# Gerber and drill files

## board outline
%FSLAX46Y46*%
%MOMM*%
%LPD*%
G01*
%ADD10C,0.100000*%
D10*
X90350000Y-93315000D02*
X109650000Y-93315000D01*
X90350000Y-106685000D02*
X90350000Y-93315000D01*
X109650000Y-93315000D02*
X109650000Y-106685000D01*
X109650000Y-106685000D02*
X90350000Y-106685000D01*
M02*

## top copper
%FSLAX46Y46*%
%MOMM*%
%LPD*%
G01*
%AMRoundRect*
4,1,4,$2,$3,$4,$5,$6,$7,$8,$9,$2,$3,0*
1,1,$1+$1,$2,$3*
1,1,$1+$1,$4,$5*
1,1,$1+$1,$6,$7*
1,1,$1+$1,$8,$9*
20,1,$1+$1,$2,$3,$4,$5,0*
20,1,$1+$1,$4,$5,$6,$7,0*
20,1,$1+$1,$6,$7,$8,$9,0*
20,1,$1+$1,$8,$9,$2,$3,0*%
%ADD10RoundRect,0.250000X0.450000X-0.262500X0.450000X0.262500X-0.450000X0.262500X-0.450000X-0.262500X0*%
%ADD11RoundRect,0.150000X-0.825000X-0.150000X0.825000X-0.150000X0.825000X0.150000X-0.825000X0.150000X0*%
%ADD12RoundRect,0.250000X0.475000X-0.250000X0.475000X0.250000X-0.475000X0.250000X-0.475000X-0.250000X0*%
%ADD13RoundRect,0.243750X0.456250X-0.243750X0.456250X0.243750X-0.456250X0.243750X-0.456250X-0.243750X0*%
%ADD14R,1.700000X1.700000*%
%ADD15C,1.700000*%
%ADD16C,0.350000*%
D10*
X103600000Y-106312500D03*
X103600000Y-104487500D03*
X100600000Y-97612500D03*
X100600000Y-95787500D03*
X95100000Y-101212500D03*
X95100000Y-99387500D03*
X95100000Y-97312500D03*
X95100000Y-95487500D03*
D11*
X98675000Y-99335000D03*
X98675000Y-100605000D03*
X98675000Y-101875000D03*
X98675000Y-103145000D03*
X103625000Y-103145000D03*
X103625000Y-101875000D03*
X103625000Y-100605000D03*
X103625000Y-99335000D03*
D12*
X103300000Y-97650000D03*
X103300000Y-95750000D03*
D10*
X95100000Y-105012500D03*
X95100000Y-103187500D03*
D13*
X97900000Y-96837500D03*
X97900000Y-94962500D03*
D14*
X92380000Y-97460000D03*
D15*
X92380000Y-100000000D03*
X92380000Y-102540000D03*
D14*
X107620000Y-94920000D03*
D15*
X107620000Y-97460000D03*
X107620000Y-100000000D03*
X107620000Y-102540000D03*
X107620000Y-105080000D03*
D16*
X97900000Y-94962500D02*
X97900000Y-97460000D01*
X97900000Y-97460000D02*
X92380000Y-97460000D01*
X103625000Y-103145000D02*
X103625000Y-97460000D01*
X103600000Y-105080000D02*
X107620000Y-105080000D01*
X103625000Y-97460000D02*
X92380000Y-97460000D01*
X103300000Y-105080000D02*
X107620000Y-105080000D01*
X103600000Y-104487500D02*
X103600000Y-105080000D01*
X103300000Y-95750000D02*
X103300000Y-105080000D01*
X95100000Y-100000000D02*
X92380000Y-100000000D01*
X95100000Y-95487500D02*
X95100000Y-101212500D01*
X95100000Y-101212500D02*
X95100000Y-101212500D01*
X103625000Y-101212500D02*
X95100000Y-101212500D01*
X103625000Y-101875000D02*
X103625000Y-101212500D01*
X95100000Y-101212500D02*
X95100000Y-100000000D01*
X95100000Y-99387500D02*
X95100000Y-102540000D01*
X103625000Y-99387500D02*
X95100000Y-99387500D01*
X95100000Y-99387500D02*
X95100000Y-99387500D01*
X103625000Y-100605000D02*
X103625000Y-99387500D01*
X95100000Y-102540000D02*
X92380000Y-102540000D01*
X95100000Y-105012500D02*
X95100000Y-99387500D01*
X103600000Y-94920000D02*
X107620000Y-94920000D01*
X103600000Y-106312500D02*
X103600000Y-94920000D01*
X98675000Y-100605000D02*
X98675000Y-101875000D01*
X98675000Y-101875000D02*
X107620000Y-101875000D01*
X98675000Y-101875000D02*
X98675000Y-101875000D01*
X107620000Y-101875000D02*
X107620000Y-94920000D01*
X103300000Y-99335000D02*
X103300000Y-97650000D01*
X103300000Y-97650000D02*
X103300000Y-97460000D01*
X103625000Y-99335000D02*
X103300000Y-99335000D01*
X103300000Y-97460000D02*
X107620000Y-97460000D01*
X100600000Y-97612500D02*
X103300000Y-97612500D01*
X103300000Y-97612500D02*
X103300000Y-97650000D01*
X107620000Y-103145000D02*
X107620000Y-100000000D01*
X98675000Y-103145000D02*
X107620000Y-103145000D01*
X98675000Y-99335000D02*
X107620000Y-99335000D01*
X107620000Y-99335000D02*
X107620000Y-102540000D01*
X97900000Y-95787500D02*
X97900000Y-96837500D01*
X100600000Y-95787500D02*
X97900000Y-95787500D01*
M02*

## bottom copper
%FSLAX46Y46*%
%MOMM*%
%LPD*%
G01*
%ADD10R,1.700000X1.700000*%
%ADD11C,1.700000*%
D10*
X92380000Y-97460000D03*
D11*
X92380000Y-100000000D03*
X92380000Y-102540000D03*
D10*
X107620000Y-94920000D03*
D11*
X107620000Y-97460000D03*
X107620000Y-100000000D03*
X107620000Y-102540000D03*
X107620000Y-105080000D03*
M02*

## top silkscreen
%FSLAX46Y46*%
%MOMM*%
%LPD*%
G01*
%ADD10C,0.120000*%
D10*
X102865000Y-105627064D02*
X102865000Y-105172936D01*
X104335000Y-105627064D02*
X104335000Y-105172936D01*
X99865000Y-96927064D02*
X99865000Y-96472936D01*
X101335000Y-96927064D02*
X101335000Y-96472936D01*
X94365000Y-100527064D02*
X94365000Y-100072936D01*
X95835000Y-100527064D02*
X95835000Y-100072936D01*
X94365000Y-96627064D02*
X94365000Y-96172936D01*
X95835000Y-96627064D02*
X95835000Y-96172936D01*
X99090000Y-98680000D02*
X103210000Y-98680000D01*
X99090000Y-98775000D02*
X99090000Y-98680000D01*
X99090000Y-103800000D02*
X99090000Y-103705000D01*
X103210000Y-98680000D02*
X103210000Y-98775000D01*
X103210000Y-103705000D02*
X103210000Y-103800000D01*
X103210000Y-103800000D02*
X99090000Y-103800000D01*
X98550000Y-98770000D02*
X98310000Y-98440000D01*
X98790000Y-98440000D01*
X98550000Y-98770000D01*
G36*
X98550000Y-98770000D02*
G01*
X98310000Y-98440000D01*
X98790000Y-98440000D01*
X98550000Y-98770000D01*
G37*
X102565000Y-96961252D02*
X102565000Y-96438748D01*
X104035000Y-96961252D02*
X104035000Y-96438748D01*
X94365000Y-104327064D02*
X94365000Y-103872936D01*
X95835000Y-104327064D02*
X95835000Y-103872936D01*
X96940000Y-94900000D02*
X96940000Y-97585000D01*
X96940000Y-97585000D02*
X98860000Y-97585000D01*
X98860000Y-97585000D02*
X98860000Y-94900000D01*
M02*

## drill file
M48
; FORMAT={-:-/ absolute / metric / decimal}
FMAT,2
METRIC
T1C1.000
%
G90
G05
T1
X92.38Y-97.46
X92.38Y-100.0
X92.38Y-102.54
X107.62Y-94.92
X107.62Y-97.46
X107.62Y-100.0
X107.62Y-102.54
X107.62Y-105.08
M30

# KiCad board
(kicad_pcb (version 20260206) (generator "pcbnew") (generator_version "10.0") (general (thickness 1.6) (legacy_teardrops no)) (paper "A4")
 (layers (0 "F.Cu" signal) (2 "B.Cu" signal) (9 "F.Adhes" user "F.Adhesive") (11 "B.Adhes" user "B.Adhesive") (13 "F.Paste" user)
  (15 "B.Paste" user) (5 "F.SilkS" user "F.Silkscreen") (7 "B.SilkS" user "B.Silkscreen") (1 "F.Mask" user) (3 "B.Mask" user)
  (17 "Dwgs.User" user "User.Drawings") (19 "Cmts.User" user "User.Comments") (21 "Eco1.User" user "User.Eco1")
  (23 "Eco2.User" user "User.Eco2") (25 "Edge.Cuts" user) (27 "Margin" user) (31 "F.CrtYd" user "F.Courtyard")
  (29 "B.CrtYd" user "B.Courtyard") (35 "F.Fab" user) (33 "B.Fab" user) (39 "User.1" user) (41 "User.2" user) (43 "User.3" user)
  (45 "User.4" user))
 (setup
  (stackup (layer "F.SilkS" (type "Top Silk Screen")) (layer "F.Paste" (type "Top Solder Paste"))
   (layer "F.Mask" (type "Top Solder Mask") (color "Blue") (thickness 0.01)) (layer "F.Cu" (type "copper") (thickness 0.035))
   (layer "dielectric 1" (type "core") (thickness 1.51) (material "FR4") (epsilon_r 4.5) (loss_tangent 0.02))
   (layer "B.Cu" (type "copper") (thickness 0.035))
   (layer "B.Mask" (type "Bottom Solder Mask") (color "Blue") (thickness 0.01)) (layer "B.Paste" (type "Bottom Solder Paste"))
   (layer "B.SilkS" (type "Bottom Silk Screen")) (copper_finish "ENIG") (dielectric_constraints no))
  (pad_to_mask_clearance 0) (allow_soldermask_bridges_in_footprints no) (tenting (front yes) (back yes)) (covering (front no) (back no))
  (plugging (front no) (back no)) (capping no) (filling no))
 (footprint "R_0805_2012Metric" (layer "F.Cu") (at 103.6 105.4 90)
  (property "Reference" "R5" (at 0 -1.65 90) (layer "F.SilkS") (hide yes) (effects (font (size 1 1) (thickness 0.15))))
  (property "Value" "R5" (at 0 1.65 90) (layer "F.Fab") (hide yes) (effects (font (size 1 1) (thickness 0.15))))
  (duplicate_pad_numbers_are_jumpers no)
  (fp_line (start -0.227064 -0.735) (end 0.227064 -0.735) (stroke (width 0.12) (type solid)) (layer "F.SilkS"))
  (fp_line (start -0.227064 0.735) (end 0.227064 0.735) (stroke (width 0.12) (type solid)) (layer "F.SilkS"))
  (pad "1" smd roundrect (at -0.9125 0 90) (size 1.025 1.4) (layers "F.Cu" "F.Mask" "F.Paste") (roundrect_rratio 0.243902) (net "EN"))
  (pad "2" smd roundrect (at 0.9125 0 90) (size 1.025 1.4) (layers "F.Cu" "F.Mask" "F.Paste") (roundrect_rratio 0.243902) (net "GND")))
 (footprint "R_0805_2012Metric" (layer "F.Cu") (at 100.6 96.7 90)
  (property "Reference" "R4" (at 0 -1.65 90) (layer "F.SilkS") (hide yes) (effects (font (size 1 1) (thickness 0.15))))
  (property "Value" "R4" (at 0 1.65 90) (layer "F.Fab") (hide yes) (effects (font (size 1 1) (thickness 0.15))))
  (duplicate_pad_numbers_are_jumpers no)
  (fp_line (start -0.227064 -0.735) (end 0.227064 -0.735) (stroke (width 0.12) (type solid)) (layer "F.SilkS"))
  (fp_line (start -0.227064 0.735) (end 0.227064 0.735) (stroke (width 0.12) (type solid)) (layer "F.SilkS"))
  (pad "1" smd roundrect (at -0.9125 0 90) (size 1.025 1.4) (layers "F.Cu" "F.Mask" "F.Paste") (roundrect_rratio 0.243902) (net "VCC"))
  (pad "2" smd roundrect (at 0.9125 0 90) (size 1.025 1.4) (layers "F.Cu" "F.Mask" "F.Paste") (roundrect_rratio 0.243902) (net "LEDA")))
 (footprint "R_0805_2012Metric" (layer "F.Cu") (at 95.1 100.3 90)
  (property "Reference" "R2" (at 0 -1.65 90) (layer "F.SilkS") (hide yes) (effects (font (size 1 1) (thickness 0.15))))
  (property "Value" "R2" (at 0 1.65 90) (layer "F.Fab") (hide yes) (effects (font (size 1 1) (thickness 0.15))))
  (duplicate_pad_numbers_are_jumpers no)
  (fp_line (start -0.227064 -0.735) (end 0.227064 -0.735) (stroke (width 0.12) (type solid)) (layer "F.SilkS"))
  (fp_line (start -0.227064 0.735) (end 0.227064 0.735) (stroke (width 0.12) (type solid)) (layer "F.SilkS"))
  (pad "1" smd roundrect (at -0.9125 0 90) (size 1.025 1.4) (layers "F.Cu" "F.Mask" "F.Paste") (roundrect_rratio 0.243902) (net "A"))
  (pad "2" smd roundrect (at 0.9125 0 90) (size 1.025 1.4) (layers "F.Cu" "F.Mask" "F.Paste") (roundrect_rratio 0.243902) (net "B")))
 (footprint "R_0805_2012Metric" (layer "F.Cu") (at 95.1 96.4 90)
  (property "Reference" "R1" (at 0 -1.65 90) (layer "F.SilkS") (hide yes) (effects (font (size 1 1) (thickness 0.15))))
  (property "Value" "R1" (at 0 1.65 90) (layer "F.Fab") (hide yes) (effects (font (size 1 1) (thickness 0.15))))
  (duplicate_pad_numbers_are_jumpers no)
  (fp_line (start -0.227064 -0.735) (end 0.227064 -0.735) (stroke (width 0.12) (type solid)) (layer "F.SilkS"))
  (fp_line (start -0.227064 0.735) (end 0.227064 0.735) (stroke (width 0.12) (type solid)) (layer "F.SilkS"))
  (pad "1" smd roundrect (at -0.9125 0 90) (size 1.025 1.4) (layers "F.Cu" "F.Mask" "F.Paste") (roundrect_rratio 0.243902) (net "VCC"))
  (pad "2" smd roundrect (at 0.9125 0 90) (size 1.025 1.4) (layers "F.Cu" "F.Mask" "F.Paste") (roundrect_rratio 0.243902) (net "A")))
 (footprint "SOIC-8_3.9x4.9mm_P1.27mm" (layer "F.Cu") (at 101.15 101.24)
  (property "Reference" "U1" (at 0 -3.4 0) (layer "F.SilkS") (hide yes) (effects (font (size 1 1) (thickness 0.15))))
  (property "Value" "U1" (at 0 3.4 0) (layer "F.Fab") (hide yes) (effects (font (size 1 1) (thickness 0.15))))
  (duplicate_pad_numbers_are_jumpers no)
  (fp_line (start -2.06 -2.56) (end 2.06 -2.56) (stroke (width 0.12) (type solid)) (layer "F.SilkS"))
  (fp_line (start -2.06 -2.465) (end -2.06 -2.56) (stroke (width 0.12) (type solid)) (layer "F.SilkS"))
  (fp_line (start -2.06 2.56) (end -2.06 2.465) (stroke (width 0.12) (type solid)) (layer "F.SilkS"))
  (fp_line (start 2.06 -2.56) (end 2.06 -2.465) (stroke (width 0.12) (type solid)) (layer "F.SilkS"))
  (fp_line (start 2.06 2.465) (end 2.06 2.56) (stroke (width 0.12) (type solid)) (layer "F.SilkS"))
  (fp_line (start 2.06 2.56) (end -2.06 2.56) (stroke (width 0.12) (type solid)) (layer "F.SilkS"))
  (fp_poly (pts (xy -2.6 -2.47) (xy -2.84 -2.8) (xy -2.36 -2.8)) (stroke (width 0.12) (type solid)) (fill yes) (layer "F.SilkS"))
  (pad "1" smd roundrect (at -2.475 -1.905) (size 1.95 0.6) (layers "F.Cu" "F.Mask" "F.Paste") (roundrect_rratio 0.25) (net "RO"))
  (pad "2" smd roundrect (at -2.475 -0.635) (size 1.95 0.6) (layers "F.Cu" "F.Mask" "F.Paste") (roundrect_rratio 0.25) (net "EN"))
  (pad "3" smd roundrect (at -2.475 0.635) (size 1.95 0.6) (layers "F.Cu" "F.Mask" "F.Paste") (roundrect_rratio 0.25) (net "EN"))
  (pad "4" smd roundrect (at -2.475 1.905) (size 1.95 0.6) (layers "F.Cu" "F.Mask" "F.Paste") (roundrect_rratio 0.25) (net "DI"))
  (pad "5" smd roundrect (at 2.475 1.905) (size 1.95 0.6) (layers "F.Cu" "F.Mask" "F.Paste") (roundrect_rratio 0.25) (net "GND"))
  (pad "6" smd roundrect (at 2.475 0.635) (size 1.95 0.6) (layers "F.Cu" "F.Mask" "F.Paste") (roundrect_rratio 0.25) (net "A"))
  (pad "7" smd roundrect (at 2.475 -0.635) (size 1.95 0.6) (layers "F.Cu" "F.Mask" "F.Paste") (roundrect_rratio 0.25) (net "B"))
  (pad "8" smd roundrect (at 2.475 -1.905) (size 1.95 0.6) (layers "F.Cu" "F.Mask" "F.Paste") (roundrect_rratio 0.25) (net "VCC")))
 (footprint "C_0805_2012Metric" (layer "F.Cu") (at 103.3 96.7 90)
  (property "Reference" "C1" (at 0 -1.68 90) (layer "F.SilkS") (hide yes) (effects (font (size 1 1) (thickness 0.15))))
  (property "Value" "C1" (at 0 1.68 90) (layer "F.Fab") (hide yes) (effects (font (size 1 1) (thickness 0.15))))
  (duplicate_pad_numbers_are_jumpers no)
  (fp_line (start -0.261252 -0.735) (end 0.261252 -0.735) (stroke (width 0.12) (type solid)) (layer "F.SilkS"))
  (fp_line (start -0.261252 0.735) (end 0.261252 0.735) (stroke (width 0.12) (type solid)) (layer "F.SilkS"))
  (pad "1" smd roundrect (at -0.95 0 90) (size 1 1.45) (layers "F.Cu" "F.Mask" "F.Paste") (roundrect_rratio 0.25) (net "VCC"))
  (pad "2" smd roundrect (at 0.95 0 90) (size 1 1.45) (layers "F.Cu" "F.Mask" "F.Paste") (roundrect_rratio 0.25) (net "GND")))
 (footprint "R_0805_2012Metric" (layer "F.Cu") (at 95.1 104.1 90)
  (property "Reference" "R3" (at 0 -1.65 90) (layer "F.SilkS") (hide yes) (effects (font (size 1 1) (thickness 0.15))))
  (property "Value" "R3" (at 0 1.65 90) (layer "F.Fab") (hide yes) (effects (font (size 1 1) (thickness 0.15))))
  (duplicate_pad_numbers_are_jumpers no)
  (fp_line (start -0.227064 -0.735) (end 0.227064 -0.735) (stroke (width 0.12) (type solid)) (layer "F.SilkS"))
  (fp_line (start -0.227064 0.735) (end 0.227064 0.735) (stroke (width 0.12) (type solid)) (layer "F.SilkS"))
  (pad "1" smd roundrect (at -0.9125 0 90) (size 1.025 1.4) (layers "F.Cu" "F.Mask" "F.Paste") (roundrect_rratio 0.243902) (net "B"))
  (pad "2" smd roundrect (at 0.9125 0 90) (size 1.025 1.4) (layers "F.Cu" "F.Mask" "F.Paste") (roundrect_rratio 0.243902) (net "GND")))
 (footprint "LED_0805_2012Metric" (layer "F.Cu") (at 97.9 95.9 90)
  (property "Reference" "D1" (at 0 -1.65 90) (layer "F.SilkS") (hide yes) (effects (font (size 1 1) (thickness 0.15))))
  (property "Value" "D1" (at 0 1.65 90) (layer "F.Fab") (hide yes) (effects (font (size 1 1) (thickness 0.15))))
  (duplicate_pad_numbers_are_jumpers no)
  (fp_line (start 1 -0.96) (end -1.685 -0.96) (stroke (width 0.12) (type solid)) (layer "F.SilkS"))
  (fp_line (start -1.685 -0.96) (end -1.685 0.96) (stroke (width 0.12) (type solid)) (layer "F.SilkS"))
  (fp_line (start -1.685 0.96) (end 1 0.96) (stroke (width 0.12) (type solid)) (layer "F.SilkS"))
  (pad "1" smd roundrect (at -0.9375 0 90) (size 0.975 1.4) (layers "F.Cu" "F.Mask" "F.Paste") (roundrect_rratio 0.25) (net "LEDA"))
  (pad "2" smd roundrect (at 0.9375 0 90) (size 0.975 1.4) (layers "F.Cu" "F.Mask" "F.Paste") (roundrect_rratio 0.25) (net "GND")))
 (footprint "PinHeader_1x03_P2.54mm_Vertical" (layer "B.Cu") (at 92.38 97.46 180)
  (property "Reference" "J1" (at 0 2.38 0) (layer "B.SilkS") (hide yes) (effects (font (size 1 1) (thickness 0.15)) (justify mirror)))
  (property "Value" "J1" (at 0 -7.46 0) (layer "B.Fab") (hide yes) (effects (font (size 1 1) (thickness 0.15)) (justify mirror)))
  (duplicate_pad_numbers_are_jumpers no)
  (pad "1" thru_hole rect (at 0 0 180) (size 1.7 1.7) (drill 1) (layers "*.Cu" "*.Mask") (remove_unused_layers no) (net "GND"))
  (pad "2" thru_hole circle (at 0 -2.54 180) (size 1.7 1.7) (drill 1) (layers "*.Cu" "*.Mask") (remove_unused_layers no) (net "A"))
  (pad "3" thru_hole circle (at 0 -5.08 180) (size 1.7 1.7) (drill 1) (layers "*.Cu" "*.Mask") (remove_unused_layers no) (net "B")))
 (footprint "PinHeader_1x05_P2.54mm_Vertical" (layer "B.Cu") (at 107.62 94.92 180)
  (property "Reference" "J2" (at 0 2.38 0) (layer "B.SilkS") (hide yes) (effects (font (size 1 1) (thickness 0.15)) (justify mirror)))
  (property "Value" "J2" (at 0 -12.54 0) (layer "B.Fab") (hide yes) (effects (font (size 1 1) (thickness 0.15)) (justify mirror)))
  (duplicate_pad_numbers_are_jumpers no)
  (pad "1" thru_hole rect (at 0 0 180) (size 1.7 1.7) (drill 1) (layers "*.Cu" "*.Mask") (remove_unused_layers no) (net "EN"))
  (pad "2" thru_hole circle (at 0 -2.54 180) (size 1.7 1.7) (drill 1) (layers "*.Cu" "*.Mask") (remove_unused_layers no) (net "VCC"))
  (pad "3" thru_hole circle (at 0 -5.08 180) (size 1.7 1.7) (drill 1) (layers "*.Cu" "*.Mask") (remove_unused_layers no) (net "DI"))
  (pad "4" thru_hole circle (at 0 -7.62 180) (size 1.7 1.7) (drill 1) (layers "*.Cu" "*.Mask") (remove_unused_layers no) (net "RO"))
  (pad "5" thru_hole circle (at 0 -10.16 180) (size 1.7 1.7) (drill 1) (layers "*.Cu" "*.Mask") (remove_unused_layers no) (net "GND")))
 (gr_line (start 90.35 93.315) (end 109.65 93.315) (stroke (width 0.1) (type default)) (layer "Edge.Cuts"))
 (gr_line (start 90.35 106.685) (end 90.35 93.315) (stroke (width 0.1) (type default)) (layer "Edge.Cuts"))
 (gr_line (start 109.65 93.315) (end 109.65 106.685) (stroke (width 0.1) (type default)) (layer "Edge.Cuts"))
 (gr_line (start 109.65 106.685) (end 90.35 106.685) (stroke (width 0.1) (type default)) (layer "Edge.Cuts"))
 (segment (start 97.9 94.9625) (end 97.9 97.46) (width 0.35) (layer "F.Cu") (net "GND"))
 (segment (start 97.9 97.46) (end 92.38 97.46) (width 0.35) (layer "F.Cu") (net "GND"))
 (segment (start 103.625 103.145) (end 103.625 97.46) (width 0.35) (layer "F.Cu") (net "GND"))
 (segment (start 103.6 105.08) (end 107.62 105.08) (width 0.35) (layer "F.Cu") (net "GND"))
 (segment (start 103.625 97.46) (end 92.38 97.46) (width 0.35) (layer "F.Cu") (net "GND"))
 (segment (start 103.3 105.08) (end 107.62 105.08) (width 0.35) (layer "F.Cu") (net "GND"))
 (segment (start 103.6 104.4875) (end 103.6 105.08) (width 0.35) (layer "F.Cu") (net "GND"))
 (segment (start 103.3 95.75) (end 103.3 105.08) (width 0.35) (layer "F.Cu") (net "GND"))
 (segment (start 95.1 100) (end 92.38 100) (width 0.35) (layer "F.Cu") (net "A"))
 (segment (start 95.1 95.4875) (end 95.1 101.2125) (width 0.35) (layer "F.Cu") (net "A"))
 (segment (start 95.1 101.2125) (end 95.1 101.2125) (width 0.35) (layer "F.Cu") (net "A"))
 (segment (start 103.625 101.2125) (end 95.1 101.2125) (width 0.35) (layer "F.Cu") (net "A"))
 (segment (start 103.625 101.875) (end 103.625 101.2125) (width 0.35) (layer "F.Cu") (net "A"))
 (segment (start 95.1 101.2125) (end 95.1 100) (width 0.35) (layer "F.Cu") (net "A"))
 (segment (start 95.1 99.3875) (end 95.1 102.54) (width 0.35) (layer "F.Cu") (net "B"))
 (segment (start 103.625 99.3875) (end 95.1 99.3875) (width 0.35) (layer "F.Cu") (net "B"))
 (segment (start 95.1 99.3875) (end 95.1 99.3875) (width 0.35) (layer "F.Cu") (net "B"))
 (segment (start 103.625 100.605) (end 103.625 99.3875) (width 0.35) (layer "F.Cu") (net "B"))
 (segment (start 95.1 102.54) (end 92.38 102.54) (width 0.35) (layer "F.Cu") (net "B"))
 (segment (start 95.1 105.0125) (end 95.1 99.3875) (width 0.35) (layer "F.Cu") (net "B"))
 (segment (start 103.6 94.92) (end 107.62 94.92) (width 0.35) (layer "F.Cu") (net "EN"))
 (segment (start 103.6 106.3125) (end 103.6 94.92) (width 0.35) (layer "F.Cu") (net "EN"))
 (segment (start 98.675 100.605) (end 98.675 101.875) (width 0.35) (layer "F.Cu") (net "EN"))
 (segment (start 98.675 101.875) (end 107.62 101.875) (width 0.35) (layer "F.Cu") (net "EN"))
 (segment (start 98.675 101.875) (end 98.675 101.875) (width 0.35) (layer "F.Cu") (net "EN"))
 (segment (start 107.62 101.875) (end 107.62 94.92) (width 0.35) (layer "F.Cu") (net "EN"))
 (segment (start 103.3 99.335) (end 103.3 97.65) (width 0.35) (layer "F.Cu") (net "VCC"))
 (segment (start 103.3 97.65) (end 103.3 97.46) (width 0.35) (layer "F.Cu") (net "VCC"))
 (segment (start 103.625 99.335) (end 103.3 99.335) (width 0.35) (layer "F.Cu") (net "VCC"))
 (segment (start 103.3 97.46) (end 107.62 97.46) (width 0.35) (layer "F.Cu") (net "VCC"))
 (segment (start 100.6 97.6125) (end 103.3 97.6125) (width 0.35) (layer "F.Cu") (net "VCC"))
 (segment (start 103.3 97.6125) (end 103.3 97.65) (width 0.35) (layer "F.Cu") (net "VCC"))
 (segment (start 107.62 103.145) (end 107.62 100) (width 0.35) (layer "F.Cu") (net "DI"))
 (segment (start 98.675 103.145) (end 107.62 103.145) (width 0.35) (layer "F.Cu") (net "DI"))
 (segment (start 98.675 99.335) (end 107.62 99.335) (width 0.35) (layer "F.Cu") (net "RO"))
 (segment (start 107.62 99.335) (end 107.62 102.54) (width 0.35) (layer "F.Cu") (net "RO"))
 (segment (start 97.9 95.7875) (end 97.9 96.8375) (width 0.35) (layer "F.Cu") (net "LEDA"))
 (segment (start 100.6 95.7875) (end 97.9 95.7875) (width 0.35) (layer "F.Cu") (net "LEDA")))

